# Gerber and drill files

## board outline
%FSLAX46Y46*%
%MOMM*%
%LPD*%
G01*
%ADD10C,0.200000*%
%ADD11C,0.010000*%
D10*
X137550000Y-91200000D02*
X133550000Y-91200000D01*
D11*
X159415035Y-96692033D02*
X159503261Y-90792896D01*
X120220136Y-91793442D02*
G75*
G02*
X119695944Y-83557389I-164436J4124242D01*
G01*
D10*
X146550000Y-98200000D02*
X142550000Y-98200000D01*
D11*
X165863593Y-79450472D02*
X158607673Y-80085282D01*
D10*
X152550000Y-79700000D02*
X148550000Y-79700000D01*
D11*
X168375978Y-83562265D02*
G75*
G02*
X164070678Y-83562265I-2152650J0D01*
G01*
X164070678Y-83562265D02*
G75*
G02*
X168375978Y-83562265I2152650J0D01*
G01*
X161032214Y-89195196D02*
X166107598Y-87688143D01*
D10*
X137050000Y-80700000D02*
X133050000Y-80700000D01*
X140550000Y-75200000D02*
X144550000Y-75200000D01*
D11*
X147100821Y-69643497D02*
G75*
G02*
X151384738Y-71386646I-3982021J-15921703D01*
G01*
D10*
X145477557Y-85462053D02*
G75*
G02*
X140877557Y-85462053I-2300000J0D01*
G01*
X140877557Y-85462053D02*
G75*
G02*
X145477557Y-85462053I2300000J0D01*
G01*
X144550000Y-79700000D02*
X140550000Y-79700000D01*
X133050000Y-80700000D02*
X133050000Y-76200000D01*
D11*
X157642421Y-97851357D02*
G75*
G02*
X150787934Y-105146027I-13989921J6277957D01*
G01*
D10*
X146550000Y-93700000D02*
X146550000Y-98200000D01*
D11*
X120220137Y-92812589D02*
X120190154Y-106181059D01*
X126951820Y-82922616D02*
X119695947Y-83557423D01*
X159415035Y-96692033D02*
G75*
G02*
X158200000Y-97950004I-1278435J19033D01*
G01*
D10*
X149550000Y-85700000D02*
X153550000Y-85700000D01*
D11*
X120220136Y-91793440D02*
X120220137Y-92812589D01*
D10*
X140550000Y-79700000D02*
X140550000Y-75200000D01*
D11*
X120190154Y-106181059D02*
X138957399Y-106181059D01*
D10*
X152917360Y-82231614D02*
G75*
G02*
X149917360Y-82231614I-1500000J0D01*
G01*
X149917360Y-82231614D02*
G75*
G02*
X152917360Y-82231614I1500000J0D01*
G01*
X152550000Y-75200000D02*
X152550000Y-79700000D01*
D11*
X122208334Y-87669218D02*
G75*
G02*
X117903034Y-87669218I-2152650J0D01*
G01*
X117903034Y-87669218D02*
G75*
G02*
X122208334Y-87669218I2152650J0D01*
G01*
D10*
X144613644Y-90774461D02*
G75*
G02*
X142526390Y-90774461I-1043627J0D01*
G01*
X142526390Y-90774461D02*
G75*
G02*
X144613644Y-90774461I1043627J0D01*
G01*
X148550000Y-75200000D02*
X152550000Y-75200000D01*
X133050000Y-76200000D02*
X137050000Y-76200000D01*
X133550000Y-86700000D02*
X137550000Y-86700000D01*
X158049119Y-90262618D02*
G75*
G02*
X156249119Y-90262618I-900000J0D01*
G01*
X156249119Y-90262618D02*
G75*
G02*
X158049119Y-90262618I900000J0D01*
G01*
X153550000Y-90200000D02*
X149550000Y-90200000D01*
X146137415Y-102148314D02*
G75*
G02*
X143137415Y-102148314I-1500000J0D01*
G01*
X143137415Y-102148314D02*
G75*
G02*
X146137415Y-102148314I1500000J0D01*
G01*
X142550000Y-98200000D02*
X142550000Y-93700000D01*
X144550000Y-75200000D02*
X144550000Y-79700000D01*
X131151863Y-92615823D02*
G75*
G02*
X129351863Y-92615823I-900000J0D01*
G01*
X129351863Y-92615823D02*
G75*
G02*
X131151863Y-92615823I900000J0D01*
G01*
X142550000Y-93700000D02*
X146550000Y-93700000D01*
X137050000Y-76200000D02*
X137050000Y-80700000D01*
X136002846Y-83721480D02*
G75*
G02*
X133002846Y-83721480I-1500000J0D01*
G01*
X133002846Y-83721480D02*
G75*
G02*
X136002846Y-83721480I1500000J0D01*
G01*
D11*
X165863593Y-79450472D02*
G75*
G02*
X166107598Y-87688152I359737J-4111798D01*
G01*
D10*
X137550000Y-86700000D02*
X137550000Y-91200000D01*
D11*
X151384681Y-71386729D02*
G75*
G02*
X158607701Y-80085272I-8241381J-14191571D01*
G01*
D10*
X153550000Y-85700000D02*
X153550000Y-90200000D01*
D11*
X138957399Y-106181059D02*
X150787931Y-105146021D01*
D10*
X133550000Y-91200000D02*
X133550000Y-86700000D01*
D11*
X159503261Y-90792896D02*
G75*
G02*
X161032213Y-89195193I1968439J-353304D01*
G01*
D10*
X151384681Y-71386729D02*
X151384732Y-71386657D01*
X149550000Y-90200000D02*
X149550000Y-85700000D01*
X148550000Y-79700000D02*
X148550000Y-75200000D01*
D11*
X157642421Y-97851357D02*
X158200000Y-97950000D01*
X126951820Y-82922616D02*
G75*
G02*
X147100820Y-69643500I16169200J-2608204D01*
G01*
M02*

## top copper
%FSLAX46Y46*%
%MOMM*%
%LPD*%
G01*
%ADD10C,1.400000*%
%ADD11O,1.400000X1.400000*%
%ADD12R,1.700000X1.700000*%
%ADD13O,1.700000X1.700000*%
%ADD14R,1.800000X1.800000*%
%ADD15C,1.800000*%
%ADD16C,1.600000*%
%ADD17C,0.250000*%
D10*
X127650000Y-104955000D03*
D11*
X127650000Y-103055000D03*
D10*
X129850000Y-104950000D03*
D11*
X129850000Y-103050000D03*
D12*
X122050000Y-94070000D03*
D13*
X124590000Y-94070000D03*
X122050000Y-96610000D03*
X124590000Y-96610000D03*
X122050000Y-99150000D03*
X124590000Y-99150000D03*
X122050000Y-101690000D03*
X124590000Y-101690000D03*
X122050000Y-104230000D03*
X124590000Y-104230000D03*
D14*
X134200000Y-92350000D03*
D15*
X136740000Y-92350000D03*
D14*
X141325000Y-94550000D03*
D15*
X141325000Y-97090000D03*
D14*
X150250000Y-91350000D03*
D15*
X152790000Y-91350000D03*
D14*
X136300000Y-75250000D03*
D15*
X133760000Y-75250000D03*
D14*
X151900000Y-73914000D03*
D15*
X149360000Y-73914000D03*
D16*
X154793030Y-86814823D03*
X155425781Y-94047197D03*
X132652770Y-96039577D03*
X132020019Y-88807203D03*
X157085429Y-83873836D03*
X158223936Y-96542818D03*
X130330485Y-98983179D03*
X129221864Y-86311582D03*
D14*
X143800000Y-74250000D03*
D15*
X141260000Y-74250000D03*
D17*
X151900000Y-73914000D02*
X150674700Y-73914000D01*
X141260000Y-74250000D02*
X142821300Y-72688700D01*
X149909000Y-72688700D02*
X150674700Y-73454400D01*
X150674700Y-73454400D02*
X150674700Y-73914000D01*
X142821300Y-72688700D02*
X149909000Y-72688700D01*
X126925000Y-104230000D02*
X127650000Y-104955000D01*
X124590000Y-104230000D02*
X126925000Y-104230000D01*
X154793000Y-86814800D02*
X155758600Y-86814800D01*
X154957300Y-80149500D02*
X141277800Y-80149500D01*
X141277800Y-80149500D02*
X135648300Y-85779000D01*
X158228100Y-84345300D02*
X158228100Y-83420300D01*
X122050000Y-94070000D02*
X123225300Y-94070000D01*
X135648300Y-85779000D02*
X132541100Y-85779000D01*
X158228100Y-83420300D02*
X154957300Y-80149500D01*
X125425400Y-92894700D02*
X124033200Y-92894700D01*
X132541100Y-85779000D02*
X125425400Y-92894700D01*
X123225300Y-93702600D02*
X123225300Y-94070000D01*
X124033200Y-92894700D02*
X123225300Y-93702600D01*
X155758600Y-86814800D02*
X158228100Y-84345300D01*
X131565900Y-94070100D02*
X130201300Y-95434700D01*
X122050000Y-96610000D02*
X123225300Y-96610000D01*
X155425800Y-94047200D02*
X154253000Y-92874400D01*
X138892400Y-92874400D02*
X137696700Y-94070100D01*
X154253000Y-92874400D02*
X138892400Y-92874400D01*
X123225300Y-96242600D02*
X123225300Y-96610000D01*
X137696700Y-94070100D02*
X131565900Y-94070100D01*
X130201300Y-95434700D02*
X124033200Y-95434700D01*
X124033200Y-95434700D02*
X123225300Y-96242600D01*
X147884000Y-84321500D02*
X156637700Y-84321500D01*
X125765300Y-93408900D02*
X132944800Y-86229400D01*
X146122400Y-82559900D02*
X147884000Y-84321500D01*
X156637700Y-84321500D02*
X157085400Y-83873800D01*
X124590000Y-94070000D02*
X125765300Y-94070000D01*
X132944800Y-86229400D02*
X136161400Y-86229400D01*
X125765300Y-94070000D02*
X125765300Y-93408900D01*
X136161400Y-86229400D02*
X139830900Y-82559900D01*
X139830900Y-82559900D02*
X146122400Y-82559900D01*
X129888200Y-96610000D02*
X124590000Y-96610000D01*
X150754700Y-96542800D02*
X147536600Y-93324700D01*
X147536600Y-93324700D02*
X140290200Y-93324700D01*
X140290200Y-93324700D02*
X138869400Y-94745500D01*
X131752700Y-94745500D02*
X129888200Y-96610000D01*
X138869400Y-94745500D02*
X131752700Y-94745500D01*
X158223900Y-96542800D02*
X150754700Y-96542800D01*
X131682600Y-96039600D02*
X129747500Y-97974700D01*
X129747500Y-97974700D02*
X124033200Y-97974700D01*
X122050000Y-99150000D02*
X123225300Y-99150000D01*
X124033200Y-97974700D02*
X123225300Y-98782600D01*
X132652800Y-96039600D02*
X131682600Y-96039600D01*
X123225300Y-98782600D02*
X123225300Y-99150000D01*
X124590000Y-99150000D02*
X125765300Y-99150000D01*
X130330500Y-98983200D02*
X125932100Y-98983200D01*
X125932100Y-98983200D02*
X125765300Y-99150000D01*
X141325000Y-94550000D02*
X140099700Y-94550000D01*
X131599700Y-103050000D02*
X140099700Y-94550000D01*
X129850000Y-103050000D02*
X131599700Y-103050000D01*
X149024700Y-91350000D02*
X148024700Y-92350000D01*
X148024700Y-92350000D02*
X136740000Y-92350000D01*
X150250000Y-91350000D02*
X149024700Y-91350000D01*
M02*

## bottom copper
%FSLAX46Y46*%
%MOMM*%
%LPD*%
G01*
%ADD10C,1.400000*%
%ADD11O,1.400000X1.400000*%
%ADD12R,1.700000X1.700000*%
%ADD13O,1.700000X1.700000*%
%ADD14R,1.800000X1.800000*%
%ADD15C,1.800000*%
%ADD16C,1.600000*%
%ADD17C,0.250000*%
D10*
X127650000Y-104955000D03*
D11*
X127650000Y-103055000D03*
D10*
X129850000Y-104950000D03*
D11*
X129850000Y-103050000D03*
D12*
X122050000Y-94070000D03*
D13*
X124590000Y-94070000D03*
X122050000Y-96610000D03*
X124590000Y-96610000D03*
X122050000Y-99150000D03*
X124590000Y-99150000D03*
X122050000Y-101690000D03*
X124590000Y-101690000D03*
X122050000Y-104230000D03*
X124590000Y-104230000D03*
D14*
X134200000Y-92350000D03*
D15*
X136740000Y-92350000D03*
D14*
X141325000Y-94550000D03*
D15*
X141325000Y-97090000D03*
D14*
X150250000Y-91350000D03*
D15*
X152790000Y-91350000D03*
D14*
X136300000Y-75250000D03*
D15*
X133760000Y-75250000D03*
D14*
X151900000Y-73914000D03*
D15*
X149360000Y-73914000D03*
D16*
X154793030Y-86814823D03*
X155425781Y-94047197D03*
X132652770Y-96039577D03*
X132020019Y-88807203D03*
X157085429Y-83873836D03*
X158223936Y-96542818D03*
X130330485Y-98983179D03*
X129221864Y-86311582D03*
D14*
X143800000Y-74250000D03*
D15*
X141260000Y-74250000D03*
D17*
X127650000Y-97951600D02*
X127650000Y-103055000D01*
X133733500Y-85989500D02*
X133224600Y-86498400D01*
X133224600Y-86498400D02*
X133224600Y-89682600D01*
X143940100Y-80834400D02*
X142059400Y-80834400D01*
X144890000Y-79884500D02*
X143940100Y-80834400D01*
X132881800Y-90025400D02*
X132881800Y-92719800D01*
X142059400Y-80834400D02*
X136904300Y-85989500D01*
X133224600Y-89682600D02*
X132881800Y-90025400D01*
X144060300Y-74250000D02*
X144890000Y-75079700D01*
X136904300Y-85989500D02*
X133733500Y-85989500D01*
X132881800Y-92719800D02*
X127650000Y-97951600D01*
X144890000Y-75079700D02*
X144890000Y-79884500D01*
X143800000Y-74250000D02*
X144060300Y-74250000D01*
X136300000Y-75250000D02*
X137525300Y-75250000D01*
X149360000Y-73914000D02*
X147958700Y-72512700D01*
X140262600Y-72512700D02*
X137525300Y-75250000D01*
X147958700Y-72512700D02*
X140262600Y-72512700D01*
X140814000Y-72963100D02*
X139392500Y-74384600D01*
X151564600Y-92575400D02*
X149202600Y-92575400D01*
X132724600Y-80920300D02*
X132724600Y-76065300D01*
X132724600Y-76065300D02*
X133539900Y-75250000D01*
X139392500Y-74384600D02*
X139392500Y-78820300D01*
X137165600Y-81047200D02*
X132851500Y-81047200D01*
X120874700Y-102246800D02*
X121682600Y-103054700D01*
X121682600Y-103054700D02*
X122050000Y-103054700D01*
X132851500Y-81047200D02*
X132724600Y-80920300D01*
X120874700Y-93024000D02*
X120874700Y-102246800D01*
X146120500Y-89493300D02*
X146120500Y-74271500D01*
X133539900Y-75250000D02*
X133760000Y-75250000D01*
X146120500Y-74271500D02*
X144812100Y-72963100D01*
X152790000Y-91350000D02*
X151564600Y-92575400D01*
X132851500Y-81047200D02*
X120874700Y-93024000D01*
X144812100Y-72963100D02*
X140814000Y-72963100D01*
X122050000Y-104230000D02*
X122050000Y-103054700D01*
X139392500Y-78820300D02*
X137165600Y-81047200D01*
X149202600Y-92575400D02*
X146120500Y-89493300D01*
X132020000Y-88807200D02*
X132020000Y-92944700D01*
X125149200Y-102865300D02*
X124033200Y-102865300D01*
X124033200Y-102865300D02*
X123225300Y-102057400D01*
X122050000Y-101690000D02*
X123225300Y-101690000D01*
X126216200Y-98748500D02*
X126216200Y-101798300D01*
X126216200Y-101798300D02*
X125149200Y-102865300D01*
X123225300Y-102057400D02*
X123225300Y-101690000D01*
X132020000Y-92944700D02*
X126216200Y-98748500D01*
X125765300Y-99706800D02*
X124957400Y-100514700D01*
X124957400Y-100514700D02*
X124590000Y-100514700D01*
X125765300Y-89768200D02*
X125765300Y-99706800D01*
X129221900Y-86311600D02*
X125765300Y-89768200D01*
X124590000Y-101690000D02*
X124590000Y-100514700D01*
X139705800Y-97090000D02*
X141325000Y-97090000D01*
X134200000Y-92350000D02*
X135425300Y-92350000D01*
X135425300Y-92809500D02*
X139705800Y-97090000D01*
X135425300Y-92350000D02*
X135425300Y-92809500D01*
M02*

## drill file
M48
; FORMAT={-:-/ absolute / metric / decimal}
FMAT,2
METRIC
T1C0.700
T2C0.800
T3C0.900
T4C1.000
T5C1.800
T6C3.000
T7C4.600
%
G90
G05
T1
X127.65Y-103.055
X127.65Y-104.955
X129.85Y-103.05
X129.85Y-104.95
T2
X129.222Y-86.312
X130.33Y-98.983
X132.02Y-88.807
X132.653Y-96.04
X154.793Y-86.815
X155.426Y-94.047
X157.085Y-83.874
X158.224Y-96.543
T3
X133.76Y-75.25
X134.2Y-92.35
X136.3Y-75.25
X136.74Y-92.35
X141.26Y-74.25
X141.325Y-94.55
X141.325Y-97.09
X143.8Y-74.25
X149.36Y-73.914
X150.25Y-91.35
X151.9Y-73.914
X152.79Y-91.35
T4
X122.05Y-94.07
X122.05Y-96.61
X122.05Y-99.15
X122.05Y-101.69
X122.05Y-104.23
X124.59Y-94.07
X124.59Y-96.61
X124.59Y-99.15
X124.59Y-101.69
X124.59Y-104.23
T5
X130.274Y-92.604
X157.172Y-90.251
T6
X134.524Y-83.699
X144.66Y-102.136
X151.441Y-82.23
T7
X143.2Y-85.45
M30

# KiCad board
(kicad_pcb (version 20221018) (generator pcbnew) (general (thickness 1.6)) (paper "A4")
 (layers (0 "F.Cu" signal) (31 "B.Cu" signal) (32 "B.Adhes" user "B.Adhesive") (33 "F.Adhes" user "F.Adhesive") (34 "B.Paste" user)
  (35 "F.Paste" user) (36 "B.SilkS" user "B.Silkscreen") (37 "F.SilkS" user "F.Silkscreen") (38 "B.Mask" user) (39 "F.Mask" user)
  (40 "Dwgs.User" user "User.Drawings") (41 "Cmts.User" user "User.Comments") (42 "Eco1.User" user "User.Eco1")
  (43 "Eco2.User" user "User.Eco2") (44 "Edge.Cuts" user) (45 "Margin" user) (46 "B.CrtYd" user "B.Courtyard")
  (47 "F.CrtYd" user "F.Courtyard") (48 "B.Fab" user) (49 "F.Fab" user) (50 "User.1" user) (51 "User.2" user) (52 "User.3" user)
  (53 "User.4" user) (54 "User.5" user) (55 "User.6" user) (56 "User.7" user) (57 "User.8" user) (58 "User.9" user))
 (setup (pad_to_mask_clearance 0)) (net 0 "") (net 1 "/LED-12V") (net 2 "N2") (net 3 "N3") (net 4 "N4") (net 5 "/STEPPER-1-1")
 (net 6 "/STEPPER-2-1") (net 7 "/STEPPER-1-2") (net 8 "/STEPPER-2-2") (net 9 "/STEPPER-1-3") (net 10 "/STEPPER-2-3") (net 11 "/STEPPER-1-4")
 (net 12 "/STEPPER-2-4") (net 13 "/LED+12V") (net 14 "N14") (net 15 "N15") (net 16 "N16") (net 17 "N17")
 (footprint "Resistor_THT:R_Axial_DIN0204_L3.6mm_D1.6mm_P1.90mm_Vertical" (layer "F.Cu") (at 127.65 104.955 90)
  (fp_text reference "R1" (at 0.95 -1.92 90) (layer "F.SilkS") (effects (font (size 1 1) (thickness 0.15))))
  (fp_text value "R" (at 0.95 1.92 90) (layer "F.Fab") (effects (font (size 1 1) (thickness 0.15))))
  (pad "1" thru_hole circle (at 0 0 90) (size 1.4 1.4) (drill 0.7) (layers "*.Cu" "*.Mask") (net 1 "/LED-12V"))
  (pad "2" thru_hole oval (at 1.9 0 90) (size 1.4 1.4) (drill 0.7) (layers "*.Cu" "*.Mask") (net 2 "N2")))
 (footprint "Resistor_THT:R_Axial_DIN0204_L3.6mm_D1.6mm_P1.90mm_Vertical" (layer "F.Cu") (at 129.85 104.95 90)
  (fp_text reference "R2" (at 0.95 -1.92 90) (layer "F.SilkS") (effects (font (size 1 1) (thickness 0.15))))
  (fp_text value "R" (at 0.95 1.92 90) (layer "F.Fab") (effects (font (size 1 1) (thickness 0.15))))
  (pad "1" thru_hole circle (at 0 0 90) (size 1.4 1.4) (drill 0.7) (layers "*.Cu" "*.Mask") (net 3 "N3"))
  (pad "2" thru_hole oval (at 1.9 0 90) (size 1.4 1.4) (drill 0.7) (layers "*.Cu" "*.Mask") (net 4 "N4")))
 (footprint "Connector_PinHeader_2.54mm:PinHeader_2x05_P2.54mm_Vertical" (layer "F.Cu") (at 122.05 94.07)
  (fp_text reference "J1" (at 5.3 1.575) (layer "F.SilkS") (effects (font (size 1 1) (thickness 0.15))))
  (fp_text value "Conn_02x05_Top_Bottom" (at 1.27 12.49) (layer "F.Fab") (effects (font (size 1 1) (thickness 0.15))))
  (pad "1" thru_hole rect (at 0 0) (size 1.7 1.7) (drill 1) (layers "*.Cu" "*.Mask") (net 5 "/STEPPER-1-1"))
  (pad "2" thru_hole oval (at 2.54 0) (size 1.7 1.7) (drill 1) (layers "*.Cu" "*.Mask") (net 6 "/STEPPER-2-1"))
  (pad "3" thru_hole oval (at 0 2.54) (size 1.7 1.7) (drill 1) (layers "*.Cu" "*.Mask") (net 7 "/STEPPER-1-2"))
  (pad "4" thru_hole oval (at 2.54 2.54) (size 1.7 1.7) (drill 1) (layers "*.Cu" "*.Mask") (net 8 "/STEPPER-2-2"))
  (pad "5" thru_hole oval (at 0 5.08) (size 1.7 1.7) (drill 1) (layers "*.Cu" "*.Mask") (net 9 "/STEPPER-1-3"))
  (pad "6" thru_hole oval (at 2.54 5.08) (size 1.7 1.7) (drill 1) (layers "*.Cu" "*.Mask") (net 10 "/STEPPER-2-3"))
  (pad "7" thru_hole oval (at 0 7.62) (size 1.7 1.7) (drill 1) (layers "*.Cu" "*.Mask") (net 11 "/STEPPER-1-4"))
  (pad "8" thru_hole oval (at 2.54 7.62) (size 1.7 1.7) (drill 1) (layers "*.Cu" "*.Mask") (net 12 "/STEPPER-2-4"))
  (pad "9" thru_hole oval (at 0 10.16) (size 1.7 1.7) (drill 1) (layers "*.Cu" "*.Mask") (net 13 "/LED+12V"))
  (pad "10" thru_hole oval (at 2.54 10.16) (size 1.7 1.7) (drill 1) (layers "*.Cu" "*.Mask") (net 1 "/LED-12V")))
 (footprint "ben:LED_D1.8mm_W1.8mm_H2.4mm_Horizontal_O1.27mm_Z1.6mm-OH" (layer "B.Cu") (at 134.2 92.35)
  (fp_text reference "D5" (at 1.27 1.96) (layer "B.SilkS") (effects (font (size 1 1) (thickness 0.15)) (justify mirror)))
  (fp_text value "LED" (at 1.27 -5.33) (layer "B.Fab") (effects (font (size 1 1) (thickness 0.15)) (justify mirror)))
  (pad "1" thru_hole rect (at 0 0) (size 1.8 1.8) (drill 0.9) (layers "*.Cu" "*.Mask") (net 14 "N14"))
  (pad "2" thru_hole circle (at 2.54 0) (size 1.8 1.8) (drill 0.9) (layers "*.Cu" "*.Mask") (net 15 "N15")))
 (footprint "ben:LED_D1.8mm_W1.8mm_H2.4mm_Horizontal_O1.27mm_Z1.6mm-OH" (layer "B.Cu") (at 141.325 94.55 -90)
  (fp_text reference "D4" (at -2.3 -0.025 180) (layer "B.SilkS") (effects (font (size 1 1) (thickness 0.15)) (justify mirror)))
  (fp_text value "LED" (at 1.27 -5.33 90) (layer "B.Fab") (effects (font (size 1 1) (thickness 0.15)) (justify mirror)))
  (pad "1" thru_hole rect (at 0 0 270) (size 1.8 1.8) (drill 0.9) (layers "*.Cu" "*.Mask") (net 4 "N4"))
  (pad "2" thru_hole circle (at 2.54 0 270) (size 1.8 1.8) (drill 0.9) (layers "*.Cu" "*.Mask") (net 14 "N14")))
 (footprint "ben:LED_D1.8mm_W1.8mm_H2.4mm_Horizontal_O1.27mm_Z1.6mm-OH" (layer "B.Cu") (at 150.25 91.35)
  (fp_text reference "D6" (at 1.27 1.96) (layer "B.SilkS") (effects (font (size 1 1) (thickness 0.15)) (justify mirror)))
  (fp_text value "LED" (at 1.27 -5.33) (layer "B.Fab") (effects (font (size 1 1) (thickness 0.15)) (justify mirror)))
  (pad "1" thru_hole rect (at 0 0) (size 1.8 1.8) (drill 0.9) (layers "*.Cu" "*.Mask") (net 15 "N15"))
  (pad "2" thru_hole circle (at 2.54 0) (size 1.8 1.8) (drill 0.9) (layers "*.Cu" "*.Mask") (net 13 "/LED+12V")))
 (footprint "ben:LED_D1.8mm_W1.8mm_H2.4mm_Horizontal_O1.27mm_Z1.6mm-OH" (layer "B.Cu") (at 136.3 75.25 180)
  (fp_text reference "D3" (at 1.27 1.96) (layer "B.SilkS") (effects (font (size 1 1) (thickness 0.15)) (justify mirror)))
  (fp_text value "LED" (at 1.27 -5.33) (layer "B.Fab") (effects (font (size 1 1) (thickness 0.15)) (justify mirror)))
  (pad "1" thru_hole rect (at 0 0 180) (size 1.8 1.8) (drill 0.9) (layers "*.Cu" "*.Mask") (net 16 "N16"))
  (pad "2" thru_hole circle (at 2.54 0 180) (size 1.8 1.8) (drill 0.9) (layers "*.Cu" "*.Mask") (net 13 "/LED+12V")))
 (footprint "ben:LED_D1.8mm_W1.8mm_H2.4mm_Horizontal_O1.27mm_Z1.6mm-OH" (layer "B.Cu") (at 151.9 73.914 180)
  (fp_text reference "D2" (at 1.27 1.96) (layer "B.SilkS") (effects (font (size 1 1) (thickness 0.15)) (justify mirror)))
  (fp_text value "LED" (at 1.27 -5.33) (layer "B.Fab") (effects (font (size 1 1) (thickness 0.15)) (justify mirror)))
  (pad "1" thru_hole rect (at 0 0 180) (size 1.8 1.8) (drill 0.9) (layers "*.Cu" "*.Mask") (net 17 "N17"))
  (pad "2" thru_hole circle (at 2.54 0 180) (size 1.8 1.8) (drill 0.9) (layers "*.Cu" "*.Mask") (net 16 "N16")))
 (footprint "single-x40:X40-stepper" (layer "B.Cu") (at 143.7229 91.4272 -175)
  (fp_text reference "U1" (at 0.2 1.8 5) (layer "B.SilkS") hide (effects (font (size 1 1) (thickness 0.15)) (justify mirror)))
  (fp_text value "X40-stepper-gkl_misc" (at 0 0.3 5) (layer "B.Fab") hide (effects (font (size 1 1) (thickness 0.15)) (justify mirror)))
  (pad "" np_thru_hole circle (at -13.5 0 185) (size 1.8 1.8) (drill 1.8) (layers "*.Cu" "*.Mask"))
  (pad "" np_thru_hole circle (at -8.49 8.49 185) (size 3 3) (drill 3) (layers "*.Cu" "*.Mask"))
  (pad "" np_thru_hole circle (at 0 -10.75 185) (size 3 3) (drill 3) (layers "*.Cu" "*.Mask"))
  (pad "" np_thru_hole circle (at 0 6 185) (size 4.6 4.6) (drill 4.6) (layers "*.Cu" "*.Mask"))
  (pad "" np_thru_hole circle (at 8.49 8.5 185) (size 3 3) (drill 3) (layers "*.Cu" "*.Mask"))
  (pad "" np_thru_hole circle (at 13.5 0 185) (size 1.8 1.8) (drill 1.8) (layers "*.Cu" "*.Mask"))
  (pad "1" thru_hole circle (at -11.43 3.63 185) (size 1.6 1.6) (drill 0.8) (layers "*.Cu" "*.Mask") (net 5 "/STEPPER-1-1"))
  (pad "2" thru_hole circle (at -11.43 -3.63 185) (size 1.6 1.6) (drill 0.8) (layers "*.Cu" "*.Mask") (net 7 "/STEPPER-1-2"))
  (pad "3" thru_hole circle (at 11.43 -3.63 185) (size 1.6 1.6) (drill 0.8) (layers "*.Cu" "*.Mask") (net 9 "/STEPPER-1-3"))
  (pad "4" thru_hole circle (at 11.43 3.63 185) (size 1.6 1.6) (drill 0.8) (layers "*.Cu" "*.Mask") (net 11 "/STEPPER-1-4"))
  (pad "5" thru_hole circle (at -13.97 6.36 185) (size 1.6 1.6) (drill 0.8) (layers "*.Cu" "*.Mask") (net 6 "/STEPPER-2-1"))
  (pad "6" thru_hole circle (at -14 -6.36 185) (size 1.6 1.6) (drill 0.8) (layers "*.Cu" "*.Mask") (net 8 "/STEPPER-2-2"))
  (pad "7" thru_hole circle (at 14 -6.36 185) (size 1.6 1.6) (drill 0.8) (layers "*.Cu" "*.Mask") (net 10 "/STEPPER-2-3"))
  (pad "8" thru_hole circle (at 14 6.36 185) (size 1.6 1.6) (drill 0.8) (layers "*.Cu" "*.Mask") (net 12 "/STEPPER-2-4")))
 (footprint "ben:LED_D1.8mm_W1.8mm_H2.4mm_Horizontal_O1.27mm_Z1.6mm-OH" (layer "B.Cu") (at 143.8 74.25 180)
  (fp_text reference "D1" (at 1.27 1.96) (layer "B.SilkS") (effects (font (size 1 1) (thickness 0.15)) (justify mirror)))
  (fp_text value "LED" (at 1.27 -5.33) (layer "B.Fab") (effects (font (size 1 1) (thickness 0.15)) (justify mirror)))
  (pad "1" thru_hole rect (at 0 0 180) (size 1.8 1.8) (drill 0.9) (layers "*.Cu" "*.Mask") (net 2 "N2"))
  (pad "2" thru_hole circle (at 2.54 0 180) (size 1.8 1.8) (drill 0.9) (layers "*.Cu" "*.Mask") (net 17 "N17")))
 (gr_line (start 137.55 91.2) (end 133.55 91.2) (stroke (width 0.2) (type solid)) (layer "Edge.Cuts"))
 (gr_line (start 159.415035 96.692033) (end 159.503261 90.792896) (stroke (width 0.01) (type solid)) (layer "Edge.Cuts"))
 (gr_arc (start 120.220136 91.793442) (mid 115.936516 87.931386) (end 119.695947 83.557423) (stroke (width 0.01) (type solid))
  (layer "Edge.Cuts"))
 (gr_line (start 146.55 98.2) (end 142.55 98.2) (stroke (width 0.2) (type solid)) (layer "Edge.Cuts"))
 (gr_line (start 165.863593 79.450472) (end 158.607673 80.085282) (stroke (width 0.01) (type solid)) (layer "Edge.Cuts"))
 (gr_line (start 152.55 79.7) (end 148.55 79.7) (stroke (width 0.2) (type solid)) (layer "Edge.Cuts"))
 (gr_circle (center 166.223328 83.562265) (end 168.375978 83.562265) (stroke (width 0.01) (type solid)) (fill none) (layer "Edge.Cuts"))
 (gr_line (start 161.032214 89.195196) (end 166.107598 87.688143) (stroke (width 0.01) (type solid)) (layer "Edge.Cuts"))
 (gr_line (start 137.05 80.7) (end 133.05 80.7) (stroke (width 0.2) (type solid)) (layer "Edge.Cuts"))
 (gr_line (start 140.55 75.2) (end 144.55 75.2) (stroke (width 0.2) (type solid)) (layer "Edge.Cuts"))
 (gr_arc (start 147.100821 69.643497) (mid 149.304488 70.363418) (end 151.384732 71.386657) (stroke (width 0.01) (type solid))
  (layer "Edge.Cuts"))
 (gr_circle (center 143.177557 85.462053) (end 140.877557 85.462053) (stroke (width 0.2) (type solid)) (fill none) (layer "Edge.Cuts"))
 (gr_line (start 144.55 79.7) (end 140.55 79.7) (stroke (width 0.2) (type solid)) (layer "Edge.Cuts"))
 (gr_line (start 133.05 80.7) (end 133.05 76.2) (stroke (width 0.2) (type solid)) (layer "Edge.Cuts"))
 (gr_arc (start 157.642421 97.851357) (mid 154.827166 102.07375) (end 150.787931 105.146021) (stroke (width 0.01) (type solid))
  (layer "Edge.Cuts"))
 (gr_line (start 146.55 93.7) (end 146.55 98.2) (stroke (width 0.2) (type solid)) (layer "Edge.Cuts"))
 (gr_line (start 120.220137 92.812589) (end 120.190154 106.181059) (stroke (width 0.01) (type solid)) (layer "Edge.Cuts"))
 (gr_line (start 126.95182 82.922616) (end 119.695947 83.557423) (stroke (width 0.01) (type solid)) (layer "Edge.Cuts"))
 (gr_arc (start 159.415035 96.692033) (mid 159.056246 97.561256) (end 158.2 97.95) (stroke (width 0.01) (type solid)) (layer "Edge.Cuts"))
 (gr_line (start 149.55 85.7) (end 153.55 85.7) (stroke (width 0.2) (type solid)) (layer "Edge.Cuts"))
 (gr_line (start 120.220136 91.79344) (end 120.220137 92.812589) (stroke (width 0.01) (type solid)) (layer "Edge.Cuts"))
 (gr_line (start 140.55 79.7) (end 140.55 75.2) (stroke (width 0.2) (type solid)) (layer "Edge.Cuts"))
 (gr_line (start 120.190154 106.181059) (end 138.957399 106.181059) (stroke (width 0.01) (type solid)) (layer "Edge.Cuts"))
 (gr_circle (center 151.41736 82.231614) (end 149.91736 82.231614) (stroke (width 0.2) (type solid)) (fill none) (layer "Edge.Cuts"))
 (gr_line (start 152.55 75.2) (end 152.55 79.7) (stroke (width 0.2) (type solid)) (layer "Edge.Cuts"))
 (gr_circle (center 120.055684 87.669218) (end 122.208334 87.669218) (stroke (width 0.01) (type solid)) (fill none) (layer "Edge.Cuts"))
 (gr_circle (center 143.570017 90.774461) (end 142.52639 90.774461) (stroke (width 0.2) (type solid)) (fill none) (layer "Edge.Cuts"))
 (gr_line (start 148.55 75.2) (end 152.55 75.2) (stroke (width 0.2) (type solid)) (layer "Edge.Cuts"))
 (gr_line (start 133.05 76.2) (end 137.05 76.2) (stroke (width 0.2) (type solid)) (layer "Edge.Cuts"))
 (gr_line (start 133.55 86.7) (end 137.55 86.7) (stroke (width 0.2) (type solid)) (layer "Edge.Cuts"))
 (gr_circle (center 157.149119 90.262618) (end 156.249119 90.262618) (stroke (width 0.2) (type solid)) (fill none) (layer "Edge.Cuts"))
 (gr_line (start 153.55 90.2) (end 149.55 90.2) (stroke (width 0.2) (type solid)) (layer "Edge.Cuts"))
 (gr_circle (center 144.637415 102.148314) (end 143.137415 102.148314) (stroke (width 0.2) (type solid)) (fill none) (layer "Edge.Cuts"))
 (gr_line (start 142.55 98.2) (end 142.55 93.7) (stroke (width 0.2) (type solid)) (layer "Edge.Cuts"))
 (gr_line (start 144.55 75.2) (end 144.55 79.7) (stroke (width 0.2) (type solid)) (layer "Edge.Cuts"))
 (gr_circle (center 130.251863 92.615823) (end 129.351863 92.615823) (stroke (width 0.2) (type solid)) (fill none) (layer "Edge.Cuts"))
 (gr_line (start 142.55 93.7) (end 146.55 93.7) (stroke (width 0.2) (type solid)) (layer "Edge.Cuts"))
 (gr_line (start 137.05 76.2) (end 137.05 80.7) (stroke (width 0.2) (type solid)) (layer "Edge.Cuts"))
 (gr_circle (center 134.502846 83.72148) (end 133.002846 83.72148) (stroke (width 0.2) (type solid)) (fill none) (layer "Edge.Cuts"))
 (gr_arc (start 165.863593 79.450472) (mid 170.349018 83.44006) (end 166.107598 87.688143) (stroke (width 0.01) (type solid))
  (layer "Edge.Cuts"))
 (gr_line (start 137.55 86.7) (end 137.55 91.2) (stroke (width 0.2) (type solid)) (layer "Edge.Cuts"))
 (gr_arc (start 151.384681 71.386729) (mid 155.768943 75.094326) (end 158.607673 80.085282) (stroke (width 0.01) (type solid))
  (layer "Edge.Cuts"))
 (gr_line (start 153.55 85.7) (end 153.55 90.2) (stroke (width 0.2) (type solid)) (layer "Edge.Cuts"))
 (gr_line (start 138.957399 106.181059) (end 150.787931 105.146021) (stroke (width 0.01) (type solid)) (layer "Edge.Cuts"))
 (gr_line (start 133.55 91.2) (end 133.55 86.7) (stroke (width 0.2) (type solid)) (layer "Edge.Cuts"))
 (gr_arc (start 159.503261 90.792896) (mid 160.026816 89.76349) (end 161.032214 89.195196) (stroke (width 0.01) (type solid))
  (layer "Edge.Cuts"))
 (gr_line (start 151.384681 71.386729) (end 151.384732 71.386657) (stroke (width 0.2) (type solid)) (layer "Edge.Cuts"))
 (gr_line (start 149.55 90.2) (end 149.55 85.7) (stroke (width 0.2) (type solid)) (layer "Edge.Cuts"))
 (gr_line (start 148.55 79.7) (end 148.55 75.2) (stroke (width 0.2) (type solid)) (layer "Edge.Cuts"))
 (gr_line (start 157.642421 97.851357) (end 158.2 97.95) (stroke (width 0.01) (type solid)) (layer "Edge.Cuts"))
 (gr_arc (start 126.95182 82.922616) (mid 134.108302 71.855416) (end 147.100821 69.643497) (stroke (width 0.01) (type solid))
  (layer "Edge.Cuts"))
 (segment (start 127.65 97.9516) (end 127.65 103.055) (width 0.25) (layer "B.Cu") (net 2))
 (segment (start 133.7335 85.9895) (end 133.2246 86.4984) (width 0.25) (layer "B.Cu") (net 2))
 (segment (start 133.2246 86.4984) (end 133.2246 89.6826) (width 0.25) (layer "B.Cu") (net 2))
 (segment (start 143.9401 80.8344) (end 142.0594 80.8344) (width 0.25) (layer "B.Cu") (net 2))
 (segment (start 144.89 79.8845) (end 143.9401 80.8344) (width 0.25) (layer "B.Cu") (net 2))
 (segment (start 132.8818 90.0254) (end 132.8818 92.7198) (width 0.25) (layer "B.Cu") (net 2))
 (segment (start 142.0594 80.8344) (end 136.9043 85.9895) (width 0.25) (layer "B.Cu") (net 2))
 (segment (start 133.2246 89.6826) (end 132.8818 90.0254) (width 0.25) (layer "B.Cu") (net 2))
 (segment (start 144.0603 74.25) (end 144.89 75.0797) (width 0.25) (layer "B.Cu") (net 2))
 (segment (start 136.9043 85.9895) (end 133.7335 85.9895) (width 0.25) (layer "B.Cu") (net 2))
 (segment (start 132.8818 92.7198) (end 127.65 97.9516) (width 0.25) (layer "B.Cu") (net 2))
 (segment (start 144.89 75.0797) (end 144.89 79.8845) (width 0.25) (layer "B.Cu") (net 2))
 (segment (start 143.8 74.25) (end 144.0603 74.25) (width 0.25) (layer "B.Cu") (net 2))
 (segment (start 151.9 73.914) (end 150.6747 73.914) (width 0.25) (layer "F.Cu") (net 17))
 (segment (start 141.26 74.25) (end 142.8213 72.6887) (width 0.25) (layer "F.Cu") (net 17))
 (segment (start 149.909 72.6887) (end 150.6747 73.4544) (width 0.25) (layer "F.Cu") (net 17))
 (segment (start 150.6747 73.4544) (end 150.6747 73.914) (width 0.25) (layer "F.Cu") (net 17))
 (segment (start 142.8213 72.6887) (end 149.909 72.6887) (width 0.25) (layer "F.Cu") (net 17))
 (segment (start 136.3 75.25) (end 137.5253 75.25) (width 0.25) (layer "B.Cu") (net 16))
 (segment (start 149.36 73.914) (end 147.9587 72.5127) (width 0.25) (layer "B.Cu") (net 16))
 (segment (start 140.2626 72.5127) (end 137.5253 75.25) (width 0.25) (layer "B.Cu") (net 16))
 (segment (start 147.9587 72.5127) (end 140.2626 72.5127) (width 0.25) (layer "B.Cu") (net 16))
 (segment (start 140.814 72.9631) (end 139.3925 74.3846) (width 0.25) (layer "B.Cu") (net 13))
 (segment (start 151.5646 92.5754) (end 149.2026 92.5754) (width 0.25) (layer "B.Cu") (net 13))
 (segment (start 132.7246 80.9203) (end 132.7246 76.0653) (width 0.25) (layer "B.Cu") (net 13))
 (segment (start 132.7246 76.0653) (end 133.5399 75.25) (width 0.25) (layer "B.Cu") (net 13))
 (segment (start 139.3925 74.3846) (end 139.3925 78.8203) (width 0.25) (layer "B.Cu") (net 13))
 (segment (start 137.1656 81.0472) (end 132.8515 81.0472) (width 0.25) (layer "B.Cu") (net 13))
 (segment (start 120.8747 102.2468) (end 121.6826 103.0547) (width 0.25) (layer "B.Cu") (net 13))
 (segment (start 121.6826 103.0547) (end 122.05 103.0547) (width 0.25) (layer "B.Cu") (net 13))
 (segment (start 132.8515 81.0472) (end 132.7246 80.9203) (width 0.25) (layer "B.Cu") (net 13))
 (segment (start 120.8747 93.024) (end 120.8747 102.2468) (width 0.25) (layer "B.Cu") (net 13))
 (segment (start 146.1205 89.4933) (end 146.1205 74.2715) (width 0.25) (layer "B.Cu") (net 13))
 (segment (start 133.5399 75.25) (end 133.76 75.25) (width 0.25) (layer "B.Cu") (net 13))
 (segment (start 146.1205 74.2715) (end 144.8121 72.9631) (width 0.25) (layer "B.Cu") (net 13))
 (segment (start 152.79 91.35) (end 151.5646 92.5754) (width 0.25) (layer "B.Cu") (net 13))
 (segment (start 132.8515 81.0472) (end 120.8747 93.024) (width 0.25) (layer "B.Cu") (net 13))
 (segment (start 144.8121 72.9631) (end 140.814 72.9631) (width 0.25) (layer "B.Cu") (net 13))
 (segment (start 122.05 104.23) (end 122.05 103.0547) (width 0.25) (layer "B.Cu") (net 13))
 (segment (start 139.3925 78.8203) (end 137.1656 81.0472) (width 0.25) (layer "B.Cu") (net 13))
 (segment (start 149.2026 92.5754) (end 146.1205 89.4933) (width 0.25) (layer "B.Cu") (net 13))
 (segment (start 126.925 104.23) (end 127.65 104.955) (width 0.25) (layer "F.Cu") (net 1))
 (segment (start 124.59 104.23) (end 126.925 104.23) (width 0.25) (layer "F.Cu") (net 1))
 (segment (start 154.793 86.8148) (end 155.7586 86.8148) (width 0.25) (layer "F.Cu") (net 5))
 (segment (start 154.9573 80.1495) (end 141.2778 80.1495) (width 0.25) (layer "F.Cu") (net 5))
 (segment (start 141.2778 80.1495) (end 135.6483 85.779) (width 0.25) (layer "F.Cu") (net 5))
 (segment (start 158.2281 84.3453) (end 158.2281 83.4203) (width 0.25) (layer "F.Cu") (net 5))
 (segment (start 122.05 94.07) (end 123.2253 94.07) (width 0.25) (layer "F.Cu") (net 5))
 (segment (start 135.6483 85.779) (end 132.5411 85.779) (width 0.25) (layer "F.Cu") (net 5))
 (segment (start 158.2281 83.4203) (end 154.9573 80.1495) (width 0.25) (layer "F.Cu") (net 5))
 (segment (start 125.4254 92.8947) (end 124.0332 92.8947) (width 0.25) (layer "F.Cu") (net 5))
 (segment (start 132.5411 85.779) (end 125.4254 92.8947) (width 0.25) (layer "F.Cu") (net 5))
 (segment (start 123.2253 93.7026) (end 123.2253 94.07) (width 0.25) (layer "F.Cu") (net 5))
 (segment (start 124.0332 92.8947) (end 123.2253 93.7026) (width 0.25) (layer "F.Cu") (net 5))
 (segment (start 155.7586 86.8148) (end 158.2281 84.3453) (width 0.25) (layer "F.Cu") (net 5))
 (segment (start 131.5659 94.0701) (end 130.2013 95.4347) (width 0.25) (layer "F.Cu") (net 7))
 (segment (start 122.05 96.61) (end 123.2253 96.61) (width 0.25) (layer "F.Cu") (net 7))
 (segment (start 155.4258 94.0472) (end 154.253 92.8744) (width 0.25) (layer "F.Cu") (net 7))
 (segment (start 138.8924 92.8744) (end 137.6967 94.0701) (width 0.25) (layer "F.Cu") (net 7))
 (segment (start 154.253 92.8744) (end 138.8924 92.8744) (width 0.25) (layer "F.Cu") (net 7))
 (segment (start 123.2253 96.2426) (end 123.2253 96.61) (width 0.25) (layer "F.Cu") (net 7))
 (segment (start 137.6967 94.0701) (end 131.5659 94.0701) (width 0.25) (layer "F.Cu") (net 7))
 (segment (start 130.2013 95.4347) (end 124.0332 95.4347) (width 0.25) (layer "F.Cu") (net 7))
 (segment (start 124.0332 95.4347) (end 123.2253 96.2426) (width 0.25) (layer "F.Cu") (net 7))
 (segment (start 147.884 84.3215) (end 156.6377 84.3215) (width 0.25) (layer "F.Cu") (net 6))
 (segment (start 125.7653 93.4089) (end 132.9448 86.2294) (width 0.25) (layer "F.Cu") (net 6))
 (segment (start 146.1224 82.5599) (end 147.884 84.3215) (width 0.25) (layer "F.Cu") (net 6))
 (segment (start 156.6377 84.3215) (end 157.0854 83.8738) (width 0.25) (layer "F.Cu") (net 6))
 (segment (start 124.59 94.07) (end 125.7653 94.07) (width 0.25) (layer "F.Cu") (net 6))
 (segment (start 132.9448 86.2294) (end 136.1614 86.2294) (width 0.25) (layer "F.Cu") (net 6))
 (segment (start 125.7653 94.07) (end 125.7653 93.4089) (width 0.25) (layer "F.Cu") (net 6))
 (segment (start 136.1614 86.2294) (end 139.8309 82.5599) (width 0.25) (layer "F.Cu") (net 6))
 (segment (start 139.8309 82.5599) (end 146.1224 82.5599) (width 0.25) (layer "F.Cu") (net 6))
 (segment (start 129.8882 96.61) (end 124.59 96.61) (width 0.25) (layer "F.Cu") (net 8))
 (segment (start 150.7547 96.5428) (end 147.5366 93.3247) (width 0.25) (layer "F.Cu") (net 8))
 (segment (start 147.5366 93.3247) (end 140.2902 93.3247) (width 0.25) (layer "F.Cu") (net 8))
 (segment (start 140.2902 93.3247) (end 138.8694 94.7455) (width 0.25) (layer "F.Cu") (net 8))
 (segment (start 131.7527 94.7455) (end 129.8882 96.61) (width 0.25) (layer "F.Cu") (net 8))
 (segment (start 138.8694 94.7455) (end 131.7527 94.7455) (width 0.25) (layer "F.Cu") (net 8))
 (segment (start 158.2239 96.5428) (end 150.7547 96.5428) (width 0.25) (layer "F.Cu") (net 8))
 (segment (start 132.02 88.8072) (end 132.02 92.9447) (width 0.25) (layer "B.Cu") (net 11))
 (segment (start 125.1492 102.8653) (end 124.0332 102.8653) (width 0.25) (layer "B.Cu") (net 11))
 (segment (start 124.0332 102.8653) (end 123.2253 102.0574) (width 0.25) (layer "B.Cu") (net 11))
 (segment (start 122.05 101.69) (end 123.2253 101.69) (width 0.25) (layer "B.Cu") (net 11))
 (segment (start 126.2162 98.7485) (end 126.2162 101.7983) (width 0.25) (layer "B.Cu") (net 11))
 (segment (start 126.2162 101.7983) (end 125.1492 102.8653) (width 0.25) (layer "B.Cu") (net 11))
 (segment (start 123.2253 102.0574) (end 123.2253 101.69) (width 0.25) (layer "B.Cu") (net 11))
 (segment (start 132.02 92.9447) (end 126.2162 98.7485) (width 0.25) (layer "B.Cu") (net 11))
 (segment (start 131.6826 96.0396) (end 129.7475 97.9747) (width 0.25) (layer "F.Cu") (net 9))
 (segment (start 129.7475 97.9747) (end 124.0332 97.9747) (width 0.25) (layer "F.Cu") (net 9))
 (segment (start 122.05 99.15) (end 123.2253 99.15) (width 0.25) (layer "F.Cu") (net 9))
 (segment (start 124.0332 97.9747) (end 123.2253 98.7826) (width 0.25) (layer "F.Cu") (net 9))
 (segment (start 132.6528 96.0396) (end 131.6826 96.0396) (width 0.25) (layer "F.Cu") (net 9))
 (segment (start 123.2253 98.7826) (end 123.2253 99.15) (width 0.25) (layer "F.Cu") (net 9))
 (segment (start 125.7653 99.7068) (end 124.9574 100.5147) (width 0.25) (layer "B.Cu") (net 12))
 (segment (start 124.9574 100.5147) (end 124.59 100.5147) (width 0.25) (layer "B.Cu") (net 12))
 (segment (start 125.7653 89.7682) (end 125.7653 99.7068) (width 0.25) (layer "B.Cu") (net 12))
 (segment (start 129.2219 86.3116) (end 125.7653 89.7682) (width 0.25) (layer "B.Cu") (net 12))
 (segment (start 124.59 101.69) (end 124.59 100.5147) (width 0.25) (layer "B.Cu") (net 12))
 (segment (start 124.59 99.15) (end 125.7653 99.15) (width 0.25) (layer "F.Cu") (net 10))
 (segment (start 130.3305 98.9832) (end 125.9321 98.9832) (width 0.25) (layer "F.Cu") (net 10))
 (segment (start 125.9321 98.9832) (end 125.7653 99.15) (width 0.25) (layer "F.Cu") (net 10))
 (segment (start 141.325 94.55) (end 140.0997 94.55) (width 0.25) (layer "F.Cu") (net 4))
 (segment (start 131.5997 103.05) (end 140.0997 94.55) (width 0.25) (layer "F.Cu") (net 4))
 (segment (start 129.85 103.05) (end 131.5997 103.05) (width 0.25) (layer "F.Cu") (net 4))
 (segment (start 139.7058 97.09) (end 141.325 97.09) (width 0.25) (layer "B.Cu") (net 14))
 (segment (start 134.2 92.35) (end 135.4253 92.35) (width 0.25) (layer "B.Cu") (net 14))
 (segment (start 135.4253 92.8095) (end 139.7058 97.09) (width 0.25) (layer "B.Cu") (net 14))
 (segment (start 135.4253 92.35) (end 135.4253 92.8095) (width 0.25) (layer "B.Cu") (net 14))
 (segment (start 149.0247 91.35) (end 148.0247 92.35) (width 0.25) (layer "F.Cu") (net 15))
 (segment (start 148.0247 92.35) (end 136.74 92.35) (width 0.25) (layer "F.Cu") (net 15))
 (segment (start 150.25 91.35) (end 149.0247 91.35) (width 0.25) (layer "F.Cu") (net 15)))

